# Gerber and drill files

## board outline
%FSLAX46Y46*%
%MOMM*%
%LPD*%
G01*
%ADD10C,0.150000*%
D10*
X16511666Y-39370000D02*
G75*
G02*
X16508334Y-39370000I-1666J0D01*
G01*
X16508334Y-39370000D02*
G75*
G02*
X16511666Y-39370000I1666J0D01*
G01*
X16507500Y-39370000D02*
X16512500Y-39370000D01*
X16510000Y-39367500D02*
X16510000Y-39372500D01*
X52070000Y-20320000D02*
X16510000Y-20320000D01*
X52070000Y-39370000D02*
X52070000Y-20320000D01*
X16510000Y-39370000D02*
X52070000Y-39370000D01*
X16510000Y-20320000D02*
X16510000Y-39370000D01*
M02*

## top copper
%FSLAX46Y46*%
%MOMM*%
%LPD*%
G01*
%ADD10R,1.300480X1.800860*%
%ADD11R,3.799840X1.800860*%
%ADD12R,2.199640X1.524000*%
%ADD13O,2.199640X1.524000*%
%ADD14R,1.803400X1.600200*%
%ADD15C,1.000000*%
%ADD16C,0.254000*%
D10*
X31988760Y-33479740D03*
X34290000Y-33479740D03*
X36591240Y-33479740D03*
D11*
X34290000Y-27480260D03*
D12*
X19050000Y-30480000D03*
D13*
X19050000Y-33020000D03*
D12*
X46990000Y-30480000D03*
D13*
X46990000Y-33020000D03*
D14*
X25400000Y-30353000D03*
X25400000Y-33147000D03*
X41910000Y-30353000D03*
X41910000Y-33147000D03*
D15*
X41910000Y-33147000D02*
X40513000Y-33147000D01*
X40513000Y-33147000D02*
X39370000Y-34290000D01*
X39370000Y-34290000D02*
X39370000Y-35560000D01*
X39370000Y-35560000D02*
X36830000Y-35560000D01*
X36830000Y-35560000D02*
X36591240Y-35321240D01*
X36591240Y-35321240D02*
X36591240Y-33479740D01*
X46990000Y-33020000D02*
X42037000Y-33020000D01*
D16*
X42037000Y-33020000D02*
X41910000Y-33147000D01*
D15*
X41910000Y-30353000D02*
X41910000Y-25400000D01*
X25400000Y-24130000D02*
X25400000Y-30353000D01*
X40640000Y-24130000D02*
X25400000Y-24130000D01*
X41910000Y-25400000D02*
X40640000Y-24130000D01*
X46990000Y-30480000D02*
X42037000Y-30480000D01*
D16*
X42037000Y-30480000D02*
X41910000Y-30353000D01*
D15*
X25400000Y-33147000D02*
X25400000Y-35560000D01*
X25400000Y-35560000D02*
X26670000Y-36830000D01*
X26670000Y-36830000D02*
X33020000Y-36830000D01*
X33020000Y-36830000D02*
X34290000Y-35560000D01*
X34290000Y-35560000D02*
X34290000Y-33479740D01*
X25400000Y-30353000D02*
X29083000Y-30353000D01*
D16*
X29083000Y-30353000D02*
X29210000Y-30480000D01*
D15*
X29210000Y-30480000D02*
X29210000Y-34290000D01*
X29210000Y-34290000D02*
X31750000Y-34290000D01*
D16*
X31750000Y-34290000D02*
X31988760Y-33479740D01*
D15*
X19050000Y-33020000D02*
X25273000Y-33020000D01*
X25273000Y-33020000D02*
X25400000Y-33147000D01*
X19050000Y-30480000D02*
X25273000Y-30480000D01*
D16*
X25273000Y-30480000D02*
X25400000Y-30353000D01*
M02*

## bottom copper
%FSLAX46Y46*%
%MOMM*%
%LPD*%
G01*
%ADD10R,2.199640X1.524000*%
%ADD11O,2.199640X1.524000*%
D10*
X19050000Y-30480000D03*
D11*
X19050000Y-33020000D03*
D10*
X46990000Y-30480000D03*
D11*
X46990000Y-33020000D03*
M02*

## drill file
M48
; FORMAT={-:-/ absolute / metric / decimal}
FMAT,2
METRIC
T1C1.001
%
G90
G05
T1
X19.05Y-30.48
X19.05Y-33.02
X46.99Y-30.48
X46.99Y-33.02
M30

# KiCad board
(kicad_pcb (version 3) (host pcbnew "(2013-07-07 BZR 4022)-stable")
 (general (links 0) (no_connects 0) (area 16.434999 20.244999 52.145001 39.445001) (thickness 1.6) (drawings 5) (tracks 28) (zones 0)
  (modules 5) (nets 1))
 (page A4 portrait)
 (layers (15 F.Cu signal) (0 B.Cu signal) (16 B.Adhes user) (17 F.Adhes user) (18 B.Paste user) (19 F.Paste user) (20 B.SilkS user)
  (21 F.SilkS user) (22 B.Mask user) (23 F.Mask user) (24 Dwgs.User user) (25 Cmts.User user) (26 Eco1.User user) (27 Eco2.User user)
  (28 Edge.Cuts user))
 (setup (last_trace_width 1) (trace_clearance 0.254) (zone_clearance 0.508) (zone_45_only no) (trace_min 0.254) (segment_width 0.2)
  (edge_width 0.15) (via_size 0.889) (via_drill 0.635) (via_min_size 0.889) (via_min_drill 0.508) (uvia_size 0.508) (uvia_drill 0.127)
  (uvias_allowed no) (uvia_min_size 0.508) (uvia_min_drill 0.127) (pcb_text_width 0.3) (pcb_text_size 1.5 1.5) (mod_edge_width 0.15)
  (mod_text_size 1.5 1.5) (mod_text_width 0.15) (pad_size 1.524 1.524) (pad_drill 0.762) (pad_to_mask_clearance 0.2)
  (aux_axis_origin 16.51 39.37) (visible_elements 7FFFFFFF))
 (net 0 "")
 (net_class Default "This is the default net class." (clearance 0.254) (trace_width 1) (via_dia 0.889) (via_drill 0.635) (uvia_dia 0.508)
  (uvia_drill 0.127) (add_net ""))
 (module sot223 (layer F.Cu) (at 34.29 30.48)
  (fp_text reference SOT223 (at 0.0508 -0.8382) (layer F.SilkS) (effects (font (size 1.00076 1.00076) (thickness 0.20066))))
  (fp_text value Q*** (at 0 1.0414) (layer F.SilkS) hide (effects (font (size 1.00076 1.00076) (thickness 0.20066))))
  (pad 1 smd rect (at -2.30124 2.99974) (size 1.30048 1.80086) (layers F.Cu F.Paste F.Mask))
  (pad 2 smd rect (at 0 2.99974) (size 1.30048 1.80086) (layers F.Cu F.Paste F.Mask))
  (pad 3 smd rect (at 2.30124 2.99974) (size 1.30048 1.80086) (layers F.Cu F.Paste F.Mask))
  (pad 4 smd rect (at 0 -2.99974) (size 3.79984 1.80086) (layers F.Cu F.Paste F.Mask)))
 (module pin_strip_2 (layer F.Cu) (at 19.05 31.75 270)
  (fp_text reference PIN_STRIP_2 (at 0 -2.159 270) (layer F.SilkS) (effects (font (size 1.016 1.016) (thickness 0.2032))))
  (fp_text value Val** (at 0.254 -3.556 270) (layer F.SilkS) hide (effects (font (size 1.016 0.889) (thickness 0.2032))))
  (pad 1 thru_hole rect (at -1.27 0 270) (size 1.524 2.19964) (drill 1.00076) (layers *.Cu *.Mask F.SilkS))
  (pad 2 thru_hole oval (at 1.27 0 270) (size 1.524 2.19964) (drill 1.00076) (layers *.Cu *.Mask F.SilkS)))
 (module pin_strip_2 (layer F.Cu) (at 46.99 31.75 270)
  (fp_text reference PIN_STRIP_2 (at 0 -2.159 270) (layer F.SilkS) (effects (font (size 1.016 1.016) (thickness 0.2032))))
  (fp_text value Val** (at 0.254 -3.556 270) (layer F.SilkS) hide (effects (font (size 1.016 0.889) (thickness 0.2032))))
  (pad 1 thru_hole rect (at -1.27 0 270) (size 1.524 2.19964) (drill 1.00076) (layers *.Cu *.Mask F.SilkS))
  (pad 2 thru_hole oval (at 1.27 0 270) (size 1.524 2.19964) (drill 1.00076) (layers *.Cu *.Mask F.SilkS)))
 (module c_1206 (layer F.Cu) (at 25.4 31.75 90)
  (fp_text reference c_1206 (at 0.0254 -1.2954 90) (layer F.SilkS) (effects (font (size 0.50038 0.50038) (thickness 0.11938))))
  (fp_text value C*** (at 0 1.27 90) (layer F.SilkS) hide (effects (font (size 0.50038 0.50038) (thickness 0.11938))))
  (pad 1 smd rect (at 1.397 0 90) (size 1.6002 1.8034) (layers F.Cu F.Paste F.Mask))
  (pad 2 smd rect (at -1.397 0 90) (size 1.6002 1.8034) (layers F.Cu F.Paste F.Mask)))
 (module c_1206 (layer F.Cu) (at 41.91 31.75 90)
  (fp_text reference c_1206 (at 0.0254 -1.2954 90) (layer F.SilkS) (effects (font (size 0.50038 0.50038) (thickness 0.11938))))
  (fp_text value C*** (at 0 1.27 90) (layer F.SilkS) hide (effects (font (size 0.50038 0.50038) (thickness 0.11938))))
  (pad 1 smd rect (at 1.397 0 90) (size 1.6002 1.8034) (layers F.Cu F.Paste F.Mask))
  (pad 2 smd rect (at -1.397 0 90) (size 1.6002 1.8034) (layers F.Cu F.Paste F.Mask)))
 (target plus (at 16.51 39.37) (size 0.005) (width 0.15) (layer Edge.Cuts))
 (gr_line (start 52.07 20.32) (end 16.51 20.32) (angle 90) (layer Edge.Cuts) (width 0.15))
 (gr_line (start 52.07 39.37) (end 52.07 20.32) (angle 90) (layer Edge.Cuts) (width 0.15))
 (gr_line (start 16.51 39.37) (end 52.07 39.37) (angle 90) (layer Edge.Cuts) (width 0.15))
 (gr_line (start 16.51 20.32) (end 16.51 39.37) (angle 90) (layer Edge.Cuts) (width 0.15))
 (segment (start 41.91 33.147) (end 40.513 33.147) (width 1) (layer F.Cu) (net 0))
 (segment (start 40.513 33.147) (end 39.37 34.29) (width 1) (layer F.Cu) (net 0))
 (segment (start 39.37 34.29) (end 39.37 35.56) (width 1) (layer F.Cu) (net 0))
 (segment (start 39.37 35.56) (end 36.83 35.56) (width 1) (layer F.Cu) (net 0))
 (segment (start 36.83 35.56) (end 36.59124 35.32124) (width 1) (layer F.Cu) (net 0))
 (segment (start 36.59124 35.32124) (end 36.59124 33.47974) (width 1) (layer F.Cu) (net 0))
 (segment (start 46.99 33.02) (end 42.037 33.02) (width 1) (layer F.Cu) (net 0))
 (segment (start 42.037 33.02) (end 41.91 33.147) (width 0.254) (layer F.Cu) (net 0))
 (segment (start 41.91 30.353) (end 41.91 25.4) (width 1) (layer F.Cu) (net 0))
 (segment (start 25.4 24.13) (end 25.4 30.353) (width 1) (layer F.Cu) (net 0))
 (segment (start 40.64 24.13) (end 25.4 24.13) (width 1) (layer F.Cu) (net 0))
 (segment (start 41.91 25.4) (end 40.64 24.13) (width 1) (layer F.Cu) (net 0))
 (segment (start 46.99 30.48) (end 42.037 30.48) (width 1) (layer F.Cu) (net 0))
 (segment (start 42.037 30.48) (end 41.91 30.353) (width 0.254) (layer F.Cu) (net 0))
 (segment (start 25.4 33.147) (end 25.4 35.56) (width 1) (layer F.Cu) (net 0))
 (segment (start 25.4 35.56) (end 26.67 36.83) (width 1) (layer F.Cu) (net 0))
 (segment (start 26.67 36.83) (end 33.02 36.83) (width 1) (layer F.Cu) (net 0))
 (segment (start 33.02 36.83) (end 34.29 35.56) (width 1) (layer F.Cu) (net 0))
 (segment (start 34.29 35.56) (end 34.29 33.47974) (width 1) (layer F.Cu) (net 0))
 (segment (start 25.4 30.353) (end 29.083 30.353) (width 1) (layer F.Cu) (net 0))
 (segment (start 29.083 30.353) (end 29.21 30.48) (width 0.254) (layer F.Cu) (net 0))
 (segment (start 29.21 30.48) (end 29.21 34.29) (width 1) (layer F.Cu) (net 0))
 (segment (start 29.21 34.29) (end 31.75 34.29) (width 1) (layer F.Cu) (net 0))
 (segment (start 31.75 34.29) (end 31.98876 33.47974) (width 0.254) (layer F.Cu) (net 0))
 (segment (start 19.05 33.02) (end 25.273 33.02) (width 1) (layer F.Cu) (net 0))
 (segment (start 25.273 33.02) (end 25.4 33.147) (width 1) (layer F.Cu) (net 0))
 (segment (start 19.05 30.48) (end 25.273 30.48) (width 1) (layer F.Cu) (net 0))
 (segment (start 25.273 30.48) (end 25.4 30.353) (width 0.254) (layer F.Cu) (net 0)))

